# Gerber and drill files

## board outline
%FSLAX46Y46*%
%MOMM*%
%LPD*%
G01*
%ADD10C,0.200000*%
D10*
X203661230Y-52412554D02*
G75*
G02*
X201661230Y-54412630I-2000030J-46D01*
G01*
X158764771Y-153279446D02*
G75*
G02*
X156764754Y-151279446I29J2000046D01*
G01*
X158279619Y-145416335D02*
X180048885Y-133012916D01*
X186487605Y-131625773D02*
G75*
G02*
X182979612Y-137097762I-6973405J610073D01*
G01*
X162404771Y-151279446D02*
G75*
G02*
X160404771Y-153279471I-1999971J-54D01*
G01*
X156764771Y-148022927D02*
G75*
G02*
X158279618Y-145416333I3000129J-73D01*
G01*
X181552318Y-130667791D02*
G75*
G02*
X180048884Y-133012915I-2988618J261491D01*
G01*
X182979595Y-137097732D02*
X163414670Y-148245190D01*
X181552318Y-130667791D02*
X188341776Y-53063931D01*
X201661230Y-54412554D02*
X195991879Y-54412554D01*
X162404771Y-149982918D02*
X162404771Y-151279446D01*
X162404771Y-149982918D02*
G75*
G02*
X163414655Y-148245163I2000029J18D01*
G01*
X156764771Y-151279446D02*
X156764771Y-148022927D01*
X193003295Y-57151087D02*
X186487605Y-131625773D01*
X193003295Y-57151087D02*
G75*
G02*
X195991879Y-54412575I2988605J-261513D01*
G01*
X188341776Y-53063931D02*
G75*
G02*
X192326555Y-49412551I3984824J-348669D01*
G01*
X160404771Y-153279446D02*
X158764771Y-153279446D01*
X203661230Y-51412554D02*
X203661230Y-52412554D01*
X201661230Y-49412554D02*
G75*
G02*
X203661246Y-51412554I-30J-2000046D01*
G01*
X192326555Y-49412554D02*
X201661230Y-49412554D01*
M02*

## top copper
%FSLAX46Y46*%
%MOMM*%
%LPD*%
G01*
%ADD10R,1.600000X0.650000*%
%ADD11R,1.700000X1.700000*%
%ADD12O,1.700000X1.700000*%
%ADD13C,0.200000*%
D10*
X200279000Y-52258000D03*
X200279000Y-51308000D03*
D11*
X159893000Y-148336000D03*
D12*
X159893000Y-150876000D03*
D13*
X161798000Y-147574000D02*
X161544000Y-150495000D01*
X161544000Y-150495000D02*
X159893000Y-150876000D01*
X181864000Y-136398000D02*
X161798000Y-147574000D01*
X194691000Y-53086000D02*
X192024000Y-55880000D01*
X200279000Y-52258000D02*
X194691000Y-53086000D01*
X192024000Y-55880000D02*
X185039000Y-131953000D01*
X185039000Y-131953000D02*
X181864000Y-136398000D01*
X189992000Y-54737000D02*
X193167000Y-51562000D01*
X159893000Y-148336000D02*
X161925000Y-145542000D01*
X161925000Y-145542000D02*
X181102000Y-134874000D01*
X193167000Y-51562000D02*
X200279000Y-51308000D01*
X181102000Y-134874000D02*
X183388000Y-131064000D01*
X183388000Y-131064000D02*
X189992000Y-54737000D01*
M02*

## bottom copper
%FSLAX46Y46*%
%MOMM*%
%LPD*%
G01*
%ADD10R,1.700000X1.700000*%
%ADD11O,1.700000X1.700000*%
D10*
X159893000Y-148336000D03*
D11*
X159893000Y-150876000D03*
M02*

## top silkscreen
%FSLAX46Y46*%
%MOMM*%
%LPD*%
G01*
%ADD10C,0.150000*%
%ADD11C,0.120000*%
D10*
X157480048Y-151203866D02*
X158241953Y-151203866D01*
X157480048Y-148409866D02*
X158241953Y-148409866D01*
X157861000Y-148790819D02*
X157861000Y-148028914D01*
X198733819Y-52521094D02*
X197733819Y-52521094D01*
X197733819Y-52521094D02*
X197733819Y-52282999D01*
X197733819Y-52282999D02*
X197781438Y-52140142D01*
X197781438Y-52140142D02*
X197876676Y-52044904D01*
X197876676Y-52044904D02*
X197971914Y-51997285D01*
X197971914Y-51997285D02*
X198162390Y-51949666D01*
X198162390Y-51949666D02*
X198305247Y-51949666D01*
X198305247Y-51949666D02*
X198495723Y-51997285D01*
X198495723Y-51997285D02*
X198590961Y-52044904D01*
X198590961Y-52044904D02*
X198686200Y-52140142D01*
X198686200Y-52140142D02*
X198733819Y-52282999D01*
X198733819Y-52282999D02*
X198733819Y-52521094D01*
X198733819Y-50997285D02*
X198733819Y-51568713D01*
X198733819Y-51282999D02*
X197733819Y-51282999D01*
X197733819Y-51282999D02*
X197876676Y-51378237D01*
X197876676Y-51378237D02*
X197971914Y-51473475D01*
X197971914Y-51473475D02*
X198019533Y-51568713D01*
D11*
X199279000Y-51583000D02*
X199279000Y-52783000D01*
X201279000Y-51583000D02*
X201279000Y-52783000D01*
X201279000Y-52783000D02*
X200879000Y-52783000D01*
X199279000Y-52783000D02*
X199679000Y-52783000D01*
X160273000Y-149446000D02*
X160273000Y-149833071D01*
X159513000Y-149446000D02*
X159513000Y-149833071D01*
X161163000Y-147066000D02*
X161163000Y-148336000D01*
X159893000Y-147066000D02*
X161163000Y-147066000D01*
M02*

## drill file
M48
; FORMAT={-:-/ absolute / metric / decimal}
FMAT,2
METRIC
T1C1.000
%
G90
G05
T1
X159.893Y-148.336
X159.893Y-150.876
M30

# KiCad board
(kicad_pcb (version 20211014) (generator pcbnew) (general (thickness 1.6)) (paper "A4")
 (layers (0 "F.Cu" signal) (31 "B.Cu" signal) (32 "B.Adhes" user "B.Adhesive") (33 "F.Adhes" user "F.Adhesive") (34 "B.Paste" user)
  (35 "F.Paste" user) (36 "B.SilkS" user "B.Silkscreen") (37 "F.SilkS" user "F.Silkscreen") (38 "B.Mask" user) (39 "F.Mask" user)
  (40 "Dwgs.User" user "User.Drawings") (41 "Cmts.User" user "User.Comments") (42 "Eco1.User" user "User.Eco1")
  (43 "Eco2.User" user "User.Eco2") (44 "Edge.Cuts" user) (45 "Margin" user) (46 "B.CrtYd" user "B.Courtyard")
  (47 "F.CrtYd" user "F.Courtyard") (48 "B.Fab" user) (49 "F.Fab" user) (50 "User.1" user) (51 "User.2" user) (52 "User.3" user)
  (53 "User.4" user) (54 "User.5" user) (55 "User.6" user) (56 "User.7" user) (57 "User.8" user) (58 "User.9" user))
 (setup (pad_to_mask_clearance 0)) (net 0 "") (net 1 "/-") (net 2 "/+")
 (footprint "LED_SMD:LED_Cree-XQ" (layer "F.Cu") (at 200.279 51.783 90)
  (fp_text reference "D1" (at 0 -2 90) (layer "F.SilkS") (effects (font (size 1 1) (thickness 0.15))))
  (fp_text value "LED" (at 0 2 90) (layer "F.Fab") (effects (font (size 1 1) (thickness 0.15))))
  (fp_line (start 0.2 -1) (end -1 -1) (layer "F.SilkS") (width 0.12))
  (fp_line (start 0.2 1) (end -1 1) (layer "F.SilkS") (width 0.12))
  (fp_line (start -1 1) (end -1 0.6) (layer "F.SilkS") (width 0.12))
  (fp_line (start -1 -1) (end -1 -0.6) (layer "F.SilkS") (width 0.12))
  (pad "1" smd rect (at -0.475 0 90) (size 0.65 1.6) (layers "F.Cu" "F.Paste" "F.Mask") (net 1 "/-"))
  (pad "2" smd rect (at 0.475 0 90) (size 0.65 1.6) (layers "F.Cu" "F.Paste" "F.Mask") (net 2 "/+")))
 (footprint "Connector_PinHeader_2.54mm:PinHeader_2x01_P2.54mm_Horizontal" (layer "F.Cu") (at 159.893 148.336 -90)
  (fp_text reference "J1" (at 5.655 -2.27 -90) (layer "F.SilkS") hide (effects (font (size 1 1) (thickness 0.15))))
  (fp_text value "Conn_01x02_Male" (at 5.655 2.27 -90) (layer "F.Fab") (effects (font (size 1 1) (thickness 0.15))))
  (fp_line (start 1.11 -0.38) (end 1.497071 -0.38) (layer "F.SilkS") (width 0.12))
  (fp_line (start 1.11 0.38) (end 1.497071 0.38) (layer "F.SilkS") (width 0.12))
  (fp_line (start -1.27 -1.27) (end 0 -1.27) (layer "F.SilkS") (width 0.12))
  (fp_line (start -1.27 0) (end -1.27 -1.27) (layer "F.SilkS") (width 0.12))
  (pad "1" thru_hole rect (at 0 0 270) (size 1.7 1.7) (drill 1) (layers *.Cu *.Mask) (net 2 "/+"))
  (pad "2" thru_hole oval (at 2.54 0 270) (size 1.7 1.7) (drill 1) (layers *.Cu *.Mask) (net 1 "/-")))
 (gr_arc (start 203.66123 52.412554) (mid 203.075444 53.826768) (end 201.66123 54.412554) (layer "Edge.Cuts") (width 0.2))
 (gr_arc (start 158.764771 153.279446) (mid 157.350558 152.693659) (end 156.764771 151.279446) (layer "Edge.Cuts") (width 0.2))
 (gr_line (start 158.279619 145.416335) (end 180.048885 133.012916) (layer "Edge.Cuts") (width 0.2))
 (gr_arc (start 186.487605 131.625773) (mid 185.407228 134.793607) (end 182.979595 137.097732) (layer "Edge.Cuts") (width 0.2))
 (gr_arc (start 162.404771 151.279446) (mid 161.818993 152.693674) (end 160.404771 153.279446) (layer "Edge.Cuts") (width 0.2))
 (gr_arc (start 156.764771 148.022927) (mid 157.171 146.515536) (end 158.279619 145.416335) (layer "Edge.Cuts") (width 0.2))
 (gr_arc (start 181.552318 130.667791) (mid 181.089299 132.025434) (end 180.048885 133.012916) (layer "Edge.Cuts") (width 0.2))
 (gr_line (start 182.979595 137.097732) (end 163.41467 148.24519) (layer "Edge.Cuts") (width 0.2))
 (gr_line (start 181.552318 130.667791) (end 188.341776 53.063931) (layer "Edge.Cuts") (width 0.2))
 (gr_line (start 201.66123 54.412554) (end 195.991879 54.412554) (layer "Edge.Cuts") (width 0.2))
 (gr_line (start 162.404771 149.982918) (end 162.404771 151.279446) (layer "Edge.Cuts") (width 0.2))
 (gr_arc (start 162.404771 149.982918) (mid 162.67558 148.977981) (end 163.41467 148.24519) (layer "Edge.Cuts") (width 0.2))
 (gr_line (start 156.764771 151.279446) (end 156.764771 148.022927) (layer "Edge.Cuts") (width 0.2))
 (gr_line (start 193.003295 57.151087) (end 186.487605 131.625773) (layer "Edge.Cuts") (width 0.2))
 (gr_arc (start 193.003295 57.151087) (mid 193.965109 55.200722) (end 195.991879 54.412554) (layer "Edge.Cuts") (width 0.2))
 (gr_arc (start 188.341776 53.063931) (mid 189.624194 50.463444) (end 192.326555 49.412554) (layer "Edge.Cuts") (width 0.2))
 (gr_line (start 160.404771 153.279446) (end 158.764771 153.279446) (layer "Edge.Cuts") (width 0.2))
 (gr_line (start 203.66123 51.412554) (end 203.66123 52.412554) (layer "Edge.Cuts") (width 0.2))
 (gr_arc (start 201.66123 49.412554) (mid 203.075444 49.99834) (end 203.66123 51.412554) (layer "Edge.Cuts") (width 0.2))
 (gr_line (start 192.326555 49.412554) (end 201.66123 49.412554) (layer "Edge.Cuts") (width 0.2))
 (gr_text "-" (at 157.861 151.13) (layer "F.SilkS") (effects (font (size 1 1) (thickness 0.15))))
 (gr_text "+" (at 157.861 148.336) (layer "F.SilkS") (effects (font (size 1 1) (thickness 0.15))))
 (segment (start 161.798 147.574) (end 161.544 150.495) (width 0.2) (layer "F.Cu") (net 1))
 (segment (start 161.544 150.495) (end 159.893 150.876) (width 0.2) (layer "F.Cu") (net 1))
 (segment (start 181.864 136.398) (end 161.798 147.574) (width 0.2) (layer "F.Cu") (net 1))
 (segment (start 194.691 53.086) (end 192.024 55.88) (width 0.2) (layer "F.Cu") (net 1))
 (segment (start 200.279 52.258) (end 194.691 53.086) (width 0.2) (layer "F.Cu") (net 1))
 (segment (start 192.024 55.88) (end 185.039 131.953) (width 0.2) (layer "F.Cu") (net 1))
 (segment (start 185.039 131.953) (end 181.864 136.398) (width 0.2) (layer "F.Cu") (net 1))
 (segment (start 189.992 54.737) (end 193.167 51.562) (width 0.2) (layer "F.Cu") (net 2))
 (segment (start 159.893 148.336) (end 161.925 145.542) (width 0.2) (layer "F.Cu") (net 2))
 (segment (start 161.925 145.542) (end 181.102 134.874) (width 0.2) (layer "F.Cu") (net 2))
 (segment (start 193.167 51.562) (end 200.279 51.308) (width 0.2) (layer "F.Cu") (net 2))
 (segment (start 181.102 134.874) (end 183.388 131.064) (width 0.2) (layer "F.Cu") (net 2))
 (segment (start 183.388 131.064) (end 189.992 54.737) (width 0.2) (layer "F.Cu") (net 2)))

